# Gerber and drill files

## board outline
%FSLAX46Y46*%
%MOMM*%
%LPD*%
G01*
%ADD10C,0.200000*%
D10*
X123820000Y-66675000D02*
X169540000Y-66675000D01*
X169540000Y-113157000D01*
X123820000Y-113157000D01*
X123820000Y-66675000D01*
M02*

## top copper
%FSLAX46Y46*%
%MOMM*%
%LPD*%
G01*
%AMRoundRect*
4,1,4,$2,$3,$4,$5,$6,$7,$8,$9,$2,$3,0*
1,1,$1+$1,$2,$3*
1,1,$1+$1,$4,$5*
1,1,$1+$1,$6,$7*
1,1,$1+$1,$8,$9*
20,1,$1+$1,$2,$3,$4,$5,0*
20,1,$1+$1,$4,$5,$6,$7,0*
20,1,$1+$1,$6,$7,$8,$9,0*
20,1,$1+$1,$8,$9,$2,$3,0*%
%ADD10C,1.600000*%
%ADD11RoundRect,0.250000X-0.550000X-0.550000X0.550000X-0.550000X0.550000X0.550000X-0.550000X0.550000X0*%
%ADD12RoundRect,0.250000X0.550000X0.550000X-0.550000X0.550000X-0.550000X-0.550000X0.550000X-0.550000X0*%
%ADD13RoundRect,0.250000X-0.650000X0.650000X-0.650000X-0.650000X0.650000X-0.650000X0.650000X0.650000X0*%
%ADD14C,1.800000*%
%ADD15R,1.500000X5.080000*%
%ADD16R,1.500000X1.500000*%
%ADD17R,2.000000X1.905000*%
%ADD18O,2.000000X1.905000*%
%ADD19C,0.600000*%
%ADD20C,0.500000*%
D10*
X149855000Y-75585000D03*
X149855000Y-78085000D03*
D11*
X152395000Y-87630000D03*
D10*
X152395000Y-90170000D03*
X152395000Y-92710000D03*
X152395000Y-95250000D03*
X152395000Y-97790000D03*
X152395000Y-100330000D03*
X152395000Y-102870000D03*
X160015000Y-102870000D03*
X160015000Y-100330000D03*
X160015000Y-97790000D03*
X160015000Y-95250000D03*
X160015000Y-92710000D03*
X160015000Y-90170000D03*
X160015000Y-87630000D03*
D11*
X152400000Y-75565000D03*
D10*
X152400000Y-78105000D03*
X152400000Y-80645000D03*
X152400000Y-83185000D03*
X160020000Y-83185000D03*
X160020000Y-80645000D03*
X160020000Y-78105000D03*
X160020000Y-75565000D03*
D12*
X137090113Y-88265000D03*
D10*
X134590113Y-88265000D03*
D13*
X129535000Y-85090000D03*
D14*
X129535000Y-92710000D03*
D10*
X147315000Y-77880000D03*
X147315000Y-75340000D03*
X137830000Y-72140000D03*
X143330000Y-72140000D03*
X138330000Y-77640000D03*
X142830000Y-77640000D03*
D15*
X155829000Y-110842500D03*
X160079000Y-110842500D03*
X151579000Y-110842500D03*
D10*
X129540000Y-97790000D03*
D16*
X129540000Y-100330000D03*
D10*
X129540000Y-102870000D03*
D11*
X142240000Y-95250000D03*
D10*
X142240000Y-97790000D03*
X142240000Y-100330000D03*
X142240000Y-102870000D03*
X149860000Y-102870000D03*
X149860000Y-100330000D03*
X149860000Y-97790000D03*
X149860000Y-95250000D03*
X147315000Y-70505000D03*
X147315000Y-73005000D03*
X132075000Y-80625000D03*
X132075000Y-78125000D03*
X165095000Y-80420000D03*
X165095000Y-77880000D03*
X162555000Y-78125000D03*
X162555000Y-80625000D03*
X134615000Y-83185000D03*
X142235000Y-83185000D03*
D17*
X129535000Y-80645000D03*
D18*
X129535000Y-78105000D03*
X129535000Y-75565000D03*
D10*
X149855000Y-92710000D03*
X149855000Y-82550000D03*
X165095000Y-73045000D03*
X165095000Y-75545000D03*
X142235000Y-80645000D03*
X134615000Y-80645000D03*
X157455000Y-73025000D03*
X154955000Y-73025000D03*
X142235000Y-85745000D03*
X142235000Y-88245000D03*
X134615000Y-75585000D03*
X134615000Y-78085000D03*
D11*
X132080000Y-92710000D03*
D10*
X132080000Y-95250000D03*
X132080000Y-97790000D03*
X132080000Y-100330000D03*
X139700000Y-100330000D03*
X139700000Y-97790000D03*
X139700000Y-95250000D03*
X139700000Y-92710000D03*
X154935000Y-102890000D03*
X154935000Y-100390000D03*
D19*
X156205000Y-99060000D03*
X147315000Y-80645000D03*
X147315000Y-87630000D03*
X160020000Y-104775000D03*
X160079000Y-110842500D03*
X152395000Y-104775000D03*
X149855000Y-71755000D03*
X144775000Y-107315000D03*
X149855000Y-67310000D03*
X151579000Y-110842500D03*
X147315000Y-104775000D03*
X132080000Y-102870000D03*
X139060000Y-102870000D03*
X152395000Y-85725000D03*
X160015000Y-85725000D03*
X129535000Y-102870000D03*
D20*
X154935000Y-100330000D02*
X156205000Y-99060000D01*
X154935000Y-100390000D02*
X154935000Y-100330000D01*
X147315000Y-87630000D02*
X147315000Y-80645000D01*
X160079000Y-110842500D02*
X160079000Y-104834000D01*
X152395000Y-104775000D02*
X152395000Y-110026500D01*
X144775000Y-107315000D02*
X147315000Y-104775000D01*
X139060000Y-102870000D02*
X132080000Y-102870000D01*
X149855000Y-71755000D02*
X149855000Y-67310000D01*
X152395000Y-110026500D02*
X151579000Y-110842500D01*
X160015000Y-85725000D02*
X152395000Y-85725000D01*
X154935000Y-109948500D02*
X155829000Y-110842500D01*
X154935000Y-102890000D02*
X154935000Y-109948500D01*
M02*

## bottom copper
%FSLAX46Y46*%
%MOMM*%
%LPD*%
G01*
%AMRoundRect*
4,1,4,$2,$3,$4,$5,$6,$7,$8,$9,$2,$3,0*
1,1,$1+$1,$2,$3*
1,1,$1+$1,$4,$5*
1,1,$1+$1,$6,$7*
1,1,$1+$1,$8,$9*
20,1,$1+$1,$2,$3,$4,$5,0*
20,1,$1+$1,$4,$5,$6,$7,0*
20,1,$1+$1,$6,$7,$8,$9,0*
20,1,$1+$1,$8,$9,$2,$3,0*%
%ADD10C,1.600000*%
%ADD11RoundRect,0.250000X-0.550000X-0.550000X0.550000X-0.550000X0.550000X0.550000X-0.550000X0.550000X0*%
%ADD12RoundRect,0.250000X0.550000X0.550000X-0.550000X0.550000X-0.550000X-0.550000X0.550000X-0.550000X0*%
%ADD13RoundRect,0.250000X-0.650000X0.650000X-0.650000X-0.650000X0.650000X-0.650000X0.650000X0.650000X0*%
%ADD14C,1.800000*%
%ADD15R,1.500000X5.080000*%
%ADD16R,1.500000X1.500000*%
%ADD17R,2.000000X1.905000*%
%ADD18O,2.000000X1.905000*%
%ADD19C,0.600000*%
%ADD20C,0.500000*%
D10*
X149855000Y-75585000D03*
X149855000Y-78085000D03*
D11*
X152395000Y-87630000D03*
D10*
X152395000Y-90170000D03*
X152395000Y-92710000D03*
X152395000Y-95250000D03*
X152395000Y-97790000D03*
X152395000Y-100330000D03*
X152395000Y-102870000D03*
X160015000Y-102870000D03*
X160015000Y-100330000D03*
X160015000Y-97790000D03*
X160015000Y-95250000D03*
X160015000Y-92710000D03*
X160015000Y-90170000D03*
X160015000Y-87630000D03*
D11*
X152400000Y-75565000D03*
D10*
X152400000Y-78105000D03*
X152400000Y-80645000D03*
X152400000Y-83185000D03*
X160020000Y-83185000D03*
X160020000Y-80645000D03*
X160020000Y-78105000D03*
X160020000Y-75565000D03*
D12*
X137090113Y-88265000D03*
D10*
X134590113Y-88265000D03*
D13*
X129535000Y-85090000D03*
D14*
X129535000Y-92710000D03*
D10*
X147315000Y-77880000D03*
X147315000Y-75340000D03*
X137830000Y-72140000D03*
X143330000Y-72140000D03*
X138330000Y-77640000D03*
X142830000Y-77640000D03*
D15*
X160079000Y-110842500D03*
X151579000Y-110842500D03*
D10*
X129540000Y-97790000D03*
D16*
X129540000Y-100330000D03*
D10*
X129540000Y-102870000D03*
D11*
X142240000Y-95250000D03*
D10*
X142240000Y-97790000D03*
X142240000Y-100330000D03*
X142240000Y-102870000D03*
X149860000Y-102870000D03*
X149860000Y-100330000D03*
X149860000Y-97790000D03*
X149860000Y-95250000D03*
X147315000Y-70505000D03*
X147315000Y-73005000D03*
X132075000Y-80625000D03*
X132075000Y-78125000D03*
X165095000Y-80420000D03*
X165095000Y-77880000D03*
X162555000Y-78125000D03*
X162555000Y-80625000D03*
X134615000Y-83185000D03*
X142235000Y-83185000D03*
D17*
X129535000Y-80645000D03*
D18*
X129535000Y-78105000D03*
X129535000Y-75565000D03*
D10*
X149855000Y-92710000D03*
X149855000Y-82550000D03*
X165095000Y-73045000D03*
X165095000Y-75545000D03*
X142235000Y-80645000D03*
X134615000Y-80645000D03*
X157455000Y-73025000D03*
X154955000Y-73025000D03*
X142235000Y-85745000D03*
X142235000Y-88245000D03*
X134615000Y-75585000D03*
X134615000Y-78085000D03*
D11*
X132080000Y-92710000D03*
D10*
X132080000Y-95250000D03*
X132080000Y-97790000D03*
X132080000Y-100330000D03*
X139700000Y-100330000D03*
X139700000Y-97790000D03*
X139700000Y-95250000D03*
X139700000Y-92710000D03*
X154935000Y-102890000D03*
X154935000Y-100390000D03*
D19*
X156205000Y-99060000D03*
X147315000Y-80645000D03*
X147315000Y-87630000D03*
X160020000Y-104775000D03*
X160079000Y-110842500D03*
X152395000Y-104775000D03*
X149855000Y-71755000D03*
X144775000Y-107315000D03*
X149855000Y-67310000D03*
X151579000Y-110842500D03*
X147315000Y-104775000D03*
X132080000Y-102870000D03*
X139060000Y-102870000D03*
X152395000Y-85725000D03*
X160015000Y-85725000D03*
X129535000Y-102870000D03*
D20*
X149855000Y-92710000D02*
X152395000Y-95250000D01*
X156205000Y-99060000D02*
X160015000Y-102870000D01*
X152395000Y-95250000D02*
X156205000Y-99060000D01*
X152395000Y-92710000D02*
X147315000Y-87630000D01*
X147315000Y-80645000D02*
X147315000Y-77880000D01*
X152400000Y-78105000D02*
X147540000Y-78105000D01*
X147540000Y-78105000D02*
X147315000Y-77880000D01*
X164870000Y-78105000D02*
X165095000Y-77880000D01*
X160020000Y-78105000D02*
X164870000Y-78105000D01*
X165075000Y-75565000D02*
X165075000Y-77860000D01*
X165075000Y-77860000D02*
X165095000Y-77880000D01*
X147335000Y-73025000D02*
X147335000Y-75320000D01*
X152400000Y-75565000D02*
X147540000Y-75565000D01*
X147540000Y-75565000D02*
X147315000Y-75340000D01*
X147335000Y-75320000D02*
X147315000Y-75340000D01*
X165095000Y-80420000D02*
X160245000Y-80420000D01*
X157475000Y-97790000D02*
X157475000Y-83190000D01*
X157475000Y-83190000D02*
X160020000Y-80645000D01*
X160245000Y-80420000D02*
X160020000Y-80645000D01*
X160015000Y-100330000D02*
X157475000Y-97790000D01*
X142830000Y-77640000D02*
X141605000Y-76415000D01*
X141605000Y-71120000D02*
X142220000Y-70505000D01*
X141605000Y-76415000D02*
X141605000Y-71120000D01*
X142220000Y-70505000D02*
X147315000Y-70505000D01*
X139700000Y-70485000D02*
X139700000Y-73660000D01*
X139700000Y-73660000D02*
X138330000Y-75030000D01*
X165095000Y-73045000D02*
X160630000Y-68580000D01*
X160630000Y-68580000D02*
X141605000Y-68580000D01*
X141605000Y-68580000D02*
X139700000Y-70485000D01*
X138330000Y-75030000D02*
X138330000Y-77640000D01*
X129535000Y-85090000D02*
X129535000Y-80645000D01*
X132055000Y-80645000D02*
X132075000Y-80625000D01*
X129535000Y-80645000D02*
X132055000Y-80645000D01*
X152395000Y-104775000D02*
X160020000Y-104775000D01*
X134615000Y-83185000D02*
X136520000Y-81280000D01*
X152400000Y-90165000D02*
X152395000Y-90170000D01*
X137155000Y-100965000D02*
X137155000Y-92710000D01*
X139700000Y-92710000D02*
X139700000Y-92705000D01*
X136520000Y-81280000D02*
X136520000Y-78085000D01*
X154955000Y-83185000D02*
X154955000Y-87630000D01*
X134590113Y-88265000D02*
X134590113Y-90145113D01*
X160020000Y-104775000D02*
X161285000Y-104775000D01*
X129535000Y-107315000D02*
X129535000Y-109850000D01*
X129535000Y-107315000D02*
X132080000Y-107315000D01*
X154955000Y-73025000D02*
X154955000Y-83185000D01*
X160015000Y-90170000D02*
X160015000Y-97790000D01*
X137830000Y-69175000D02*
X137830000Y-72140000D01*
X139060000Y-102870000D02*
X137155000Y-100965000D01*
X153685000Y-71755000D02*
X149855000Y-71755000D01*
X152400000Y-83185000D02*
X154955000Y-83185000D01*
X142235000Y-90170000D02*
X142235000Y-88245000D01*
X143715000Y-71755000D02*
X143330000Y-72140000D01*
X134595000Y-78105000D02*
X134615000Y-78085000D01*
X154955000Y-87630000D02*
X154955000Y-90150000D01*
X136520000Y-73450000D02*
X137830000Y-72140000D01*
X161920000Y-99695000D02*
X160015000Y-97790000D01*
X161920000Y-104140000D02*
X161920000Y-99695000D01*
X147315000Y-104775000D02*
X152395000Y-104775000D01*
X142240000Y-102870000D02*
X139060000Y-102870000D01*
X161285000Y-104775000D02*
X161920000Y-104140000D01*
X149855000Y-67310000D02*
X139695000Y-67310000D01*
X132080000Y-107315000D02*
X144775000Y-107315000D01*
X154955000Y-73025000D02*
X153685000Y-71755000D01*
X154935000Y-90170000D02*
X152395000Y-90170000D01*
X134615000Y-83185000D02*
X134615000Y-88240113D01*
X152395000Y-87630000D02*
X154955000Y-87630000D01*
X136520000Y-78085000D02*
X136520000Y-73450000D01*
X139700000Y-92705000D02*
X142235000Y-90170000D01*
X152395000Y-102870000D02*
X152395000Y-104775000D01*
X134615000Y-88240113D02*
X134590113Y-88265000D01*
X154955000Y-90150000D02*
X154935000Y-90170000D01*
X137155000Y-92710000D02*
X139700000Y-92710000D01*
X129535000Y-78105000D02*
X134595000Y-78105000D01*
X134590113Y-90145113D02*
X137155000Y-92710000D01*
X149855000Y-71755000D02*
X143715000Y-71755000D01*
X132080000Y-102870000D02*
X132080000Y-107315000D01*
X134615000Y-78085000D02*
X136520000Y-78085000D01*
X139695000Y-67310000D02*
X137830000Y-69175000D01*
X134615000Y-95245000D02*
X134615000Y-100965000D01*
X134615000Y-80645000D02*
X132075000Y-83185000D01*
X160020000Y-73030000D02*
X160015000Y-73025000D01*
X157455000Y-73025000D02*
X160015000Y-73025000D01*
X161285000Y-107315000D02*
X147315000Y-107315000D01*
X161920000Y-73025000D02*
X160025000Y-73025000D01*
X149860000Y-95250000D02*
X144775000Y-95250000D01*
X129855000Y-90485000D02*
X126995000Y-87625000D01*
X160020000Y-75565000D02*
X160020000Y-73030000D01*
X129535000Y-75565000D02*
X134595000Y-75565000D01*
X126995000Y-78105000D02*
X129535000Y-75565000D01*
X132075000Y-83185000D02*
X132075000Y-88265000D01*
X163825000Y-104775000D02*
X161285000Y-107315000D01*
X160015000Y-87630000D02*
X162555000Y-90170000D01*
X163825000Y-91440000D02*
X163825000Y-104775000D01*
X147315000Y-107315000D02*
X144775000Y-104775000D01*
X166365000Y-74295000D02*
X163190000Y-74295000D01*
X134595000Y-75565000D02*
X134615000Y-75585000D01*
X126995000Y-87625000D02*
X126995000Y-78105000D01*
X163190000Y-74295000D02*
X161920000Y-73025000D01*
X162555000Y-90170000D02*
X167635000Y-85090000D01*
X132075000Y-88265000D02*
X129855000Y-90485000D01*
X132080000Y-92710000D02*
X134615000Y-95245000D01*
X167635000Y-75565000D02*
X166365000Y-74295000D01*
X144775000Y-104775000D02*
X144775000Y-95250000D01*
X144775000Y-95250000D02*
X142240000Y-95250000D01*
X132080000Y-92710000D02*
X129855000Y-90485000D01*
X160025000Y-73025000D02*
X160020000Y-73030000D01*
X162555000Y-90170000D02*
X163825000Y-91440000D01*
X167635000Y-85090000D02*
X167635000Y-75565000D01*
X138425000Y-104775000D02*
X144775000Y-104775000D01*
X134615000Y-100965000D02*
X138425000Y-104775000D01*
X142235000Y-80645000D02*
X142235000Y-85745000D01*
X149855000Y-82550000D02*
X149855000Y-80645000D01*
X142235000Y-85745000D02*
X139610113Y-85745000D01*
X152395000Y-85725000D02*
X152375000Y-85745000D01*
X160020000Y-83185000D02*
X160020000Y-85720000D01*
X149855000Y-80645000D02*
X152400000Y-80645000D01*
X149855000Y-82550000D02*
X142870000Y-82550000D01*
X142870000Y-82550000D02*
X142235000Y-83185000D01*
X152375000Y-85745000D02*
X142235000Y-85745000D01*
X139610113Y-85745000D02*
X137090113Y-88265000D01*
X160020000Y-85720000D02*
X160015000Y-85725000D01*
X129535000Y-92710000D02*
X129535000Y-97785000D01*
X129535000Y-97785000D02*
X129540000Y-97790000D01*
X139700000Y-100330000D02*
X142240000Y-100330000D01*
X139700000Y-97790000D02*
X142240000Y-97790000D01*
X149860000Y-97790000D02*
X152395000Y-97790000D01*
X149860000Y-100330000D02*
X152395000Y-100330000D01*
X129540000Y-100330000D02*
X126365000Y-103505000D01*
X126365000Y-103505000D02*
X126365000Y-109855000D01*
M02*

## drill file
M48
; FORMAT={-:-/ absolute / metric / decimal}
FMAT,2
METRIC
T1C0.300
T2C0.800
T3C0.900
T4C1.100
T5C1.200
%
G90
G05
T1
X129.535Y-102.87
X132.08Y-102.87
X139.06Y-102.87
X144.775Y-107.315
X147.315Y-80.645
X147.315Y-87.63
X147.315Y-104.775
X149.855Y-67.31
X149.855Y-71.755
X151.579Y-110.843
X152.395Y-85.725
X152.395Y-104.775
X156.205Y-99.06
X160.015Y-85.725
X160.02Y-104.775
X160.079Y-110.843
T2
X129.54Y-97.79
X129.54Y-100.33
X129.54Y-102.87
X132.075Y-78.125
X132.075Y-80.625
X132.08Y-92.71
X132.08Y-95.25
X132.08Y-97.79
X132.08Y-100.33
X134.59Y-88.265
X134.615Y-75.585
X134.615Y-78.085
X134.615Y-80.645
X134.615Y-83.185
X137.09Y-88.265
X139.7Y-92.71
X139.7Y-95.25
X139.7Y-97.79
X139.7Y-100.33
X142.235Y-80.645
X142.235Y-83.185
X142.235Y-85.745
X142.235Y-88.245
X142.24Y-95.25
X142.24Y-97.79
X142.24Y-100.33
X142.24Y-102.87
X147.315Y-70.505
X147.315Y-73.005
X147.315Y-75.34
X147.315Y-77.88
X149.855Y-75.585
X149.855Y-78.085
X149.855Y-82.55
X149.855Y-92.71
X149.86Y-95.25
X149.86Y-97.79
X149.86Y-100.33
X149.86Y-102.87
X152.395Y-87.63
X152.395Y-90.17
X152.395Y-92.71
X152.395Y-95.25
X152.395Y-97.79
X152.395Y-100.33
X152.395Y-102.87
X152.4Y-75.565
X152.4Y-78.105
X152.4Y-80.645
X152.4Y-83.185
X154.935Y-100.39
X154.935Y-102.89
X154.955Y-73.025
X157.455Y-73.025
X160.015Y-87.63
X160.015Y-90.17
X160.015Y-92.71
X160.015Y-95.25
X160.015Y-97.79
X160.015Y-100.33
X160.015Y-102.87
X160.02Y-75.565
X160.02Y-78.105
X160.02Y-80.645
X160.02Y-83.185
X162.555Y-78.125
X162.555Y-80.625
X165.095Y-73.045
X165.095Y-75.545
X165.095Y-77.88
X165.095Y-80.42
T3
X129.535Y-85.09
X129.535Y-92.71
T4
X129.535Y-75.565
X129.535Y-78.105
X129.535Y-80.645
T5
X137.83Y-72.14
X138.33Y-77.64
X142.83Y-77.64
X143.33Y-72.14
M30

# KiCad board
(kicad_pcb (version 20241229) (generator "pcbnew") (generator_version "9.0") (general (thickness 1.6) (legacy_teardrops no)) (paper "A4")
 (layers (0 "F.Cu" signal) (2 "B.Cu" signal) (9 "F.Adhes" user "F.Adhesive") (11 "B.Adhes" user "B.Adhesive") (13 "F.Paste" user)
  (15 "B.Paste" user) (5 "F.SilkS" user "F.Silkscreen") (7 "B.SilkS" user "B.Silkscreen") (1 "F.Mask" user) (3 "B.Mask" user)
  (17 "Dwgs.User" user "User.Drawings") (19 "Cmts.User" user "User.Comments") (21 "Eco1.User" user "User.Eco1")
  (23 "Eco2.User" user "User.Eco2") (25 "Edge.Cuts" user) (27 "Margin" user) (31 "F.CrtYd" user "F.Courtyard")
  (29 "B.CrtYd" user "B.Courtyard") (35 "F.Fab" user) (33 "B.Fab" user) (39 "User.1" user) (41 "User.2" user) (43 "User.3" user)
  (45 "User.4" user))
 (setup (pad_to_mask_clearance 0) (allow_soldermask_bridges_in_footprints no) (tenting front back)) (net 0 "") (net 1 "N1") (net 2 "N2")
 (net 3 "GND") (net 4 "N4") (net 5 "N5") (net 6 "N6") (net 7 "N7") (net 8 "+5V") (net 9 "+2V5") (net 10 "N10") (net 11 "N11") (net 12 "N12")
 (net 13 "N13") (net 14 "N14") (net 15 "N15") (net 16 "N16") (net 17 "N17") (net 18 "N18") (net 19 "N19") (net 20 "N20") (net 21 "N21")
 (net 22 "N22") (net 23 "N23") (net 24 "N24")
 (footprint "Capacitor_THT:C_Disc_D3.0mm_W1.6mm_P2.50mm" (layer "F.Cu") (at 149.855 75.585 -90)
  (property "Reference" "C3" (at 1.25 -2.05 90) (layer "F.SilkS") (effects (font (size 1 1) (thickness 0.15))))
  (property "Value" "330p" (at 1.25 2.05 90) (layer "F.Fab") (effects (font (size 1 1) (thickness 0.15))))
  (pad "1" thru_hole circle (at 0 0 270) (size 1.6 1.6) (drill 0.8) (layers "*.Cu" "*.Mask") (remove_unused_layers no) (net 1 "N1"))
  (pad "2" thru_hole circle (at 2.5 0 270) (size 1.6 1.6) (drill 0.8) (layers "*.Cu" "*.Mask") (remove_unused_layers no) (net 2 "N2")))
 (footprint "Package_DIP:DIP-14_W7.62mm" (layer "F.Cu") (at 152.395 87.63)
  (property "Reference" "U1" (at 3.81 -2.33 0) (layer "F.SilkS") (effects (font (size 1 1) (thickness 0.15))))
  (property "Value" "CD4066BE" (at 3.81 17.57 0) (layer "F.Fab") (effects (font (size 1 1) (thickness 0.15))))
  (pad "1" thru_hole roundrect (at 0 0) (size 1.6 1.6) (drill 0.8) (layers "*.Cu" "*.Mask") (remove_unused_layers no)
   (roundrect_rratio 0.15625) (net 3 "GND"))
  (pad "2" thru_hole circle (at 0 2.54) (size 1.6 1.6) (drill 0.8) (layers "*.Cu" "*.Mask") (remove_unused_layers no) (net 3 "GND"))
  (pad "3" thru_hole circle (at 0 5.08) (size 1.6 1.6) (drill 0.8) (layers "*.Cu" "*.Mask") (remove_unused_layers no) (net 2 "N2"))
  (pad "4" thru_hole circle (at 0 7.62) (size 1.6 1.6) (drill 0.8) (layers "*.Cu" "*.Mask") (remove_unused_layers no) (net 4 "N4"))
  (pad "5" thru_hole circle (at 0 10.16) (size 1.6 1.6) (drill 0.8) (layers "*.Cu" "*.Mask") (remove_unused_layers no) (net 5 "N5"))
  (pad "6" thru_hole circle (at 0 12.7) (size 1.6 1.6) (drill 0.8) (layers "*.Cu" "*.Mask") (remove_unused_layers no) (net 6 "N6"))
  (pad "7" thru_hole circle (at 0 15.24) (size 1.6 1.6) (drill 0.8) (layers "*.Cu" "*.Mask") (remove_unused_layers no) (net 3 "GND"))
  (pad "8" thru_hole circle (at 7.62 15.24) (size 1.6 1.6) (drill 0.8) (layers "*.Cu" "*.Mask") (remove_unused_layers no) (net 4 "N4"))
  (pad "9" thru_hole circle (at 7.62 12.7) (size 1.6 1.6) (drill 0.8) (layers "*.Cu" "*.Mask") (remove_unused_layers no) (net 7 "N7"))
  (pad "10" thru_hole circle (at 7.62 10.16) (size 1.6 1.6) (drill 0.8) (layers "*.Cu" "*.Mask") (remove_unused_layers no) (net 3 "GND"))
  (pad "11" thru_hole circle (at 7.62 7.62) (size 1.6 1.6) (drill 0.8) (layers "*.Cu" "*.Mask") (remove_unused_layers no) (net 3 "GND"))
  (pad "12" thru_hole circle (at 7.62 5.08) (size 1.6 1.6) (drill 0.8) (layers "*.Cu" "*.Mask") (remove_unused_layers no) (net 3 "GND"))
  (pad "13" thru_hole circle (at 7.62 2.54) (size 1.6 1.6) (drill 0.8) (layers "*.Cu" "*.Mask") (remove_unused_layers no) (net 3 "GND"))
  (pad "14" thru_hole circle (at 7.62 0) (size 1.6 1.6) (drill 0.8) (layers "*.Cu" "*.Mask") (remove_unused_layers no) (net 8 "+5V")))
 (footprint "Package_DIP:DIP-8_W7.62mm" (layer "F.Cu") (at 152.4 75.565)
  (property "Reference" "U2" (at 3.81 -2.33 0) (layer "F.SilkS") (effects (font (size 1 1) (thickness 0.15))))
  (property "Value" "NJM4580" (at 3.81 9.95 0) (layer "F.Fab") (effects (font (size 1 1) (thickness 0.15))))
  (pad "1" thru_hole roundrect (at 0 0) (size 1.6 1.6) (drill 0.8) (layers "*.Cu" "*.Mask") (remove_unused_layers no)
   (roundrect_rratio 0.15625) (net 1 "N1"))
  (pad "2" thru_hole circle (at 0 2.54) (size 1.6 1.6) (drill 0.8) (layers "*.Cu" "*.Mask") (remove_unused_layers no) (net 2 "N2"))
  (pad "3" thru_hole circle (at 0 5.08) (size 1.6 1.6) (drill 0.8) (layers "*.Cu" "*.Mask") (remove_unused_layers no) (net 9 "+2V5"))
  (pad "4" thru_hole circle (at 0 7.62) (size 1.6 1.6) (drill 0.8) (layers "*.Cu" "*.Mask") (remove_unused_layers no) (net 3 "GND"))
  (pad "5" thru_hole circle (at 7.62 7.62) (size 1.6 1.6) (drill 0.8) (layers "*.Cu" "*.Mask") (remove_unused_layers no) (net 9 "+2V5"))
  (pad "6" thru_hole circle (at 7.62 5.08) (size 1.6 1.6) (drill 0.8) (layers "*.Cu" "*.Mask") (remove_unused_layers no) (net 7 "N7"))
  (pad "7" thru_hole circle (at 7.62 2.54) (size 1.6 1.6) (drill 0.8) (layers "*.Cu" "*.Mask") (remove_unused_layers no) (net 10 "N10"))
  (pad "8" thru_hole circle (at 7.62 0) (size 1.6 1.6) (drill 0.8) (layers "*.Cu" "*.Mask") (remove_unused_layers no) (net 8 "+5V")))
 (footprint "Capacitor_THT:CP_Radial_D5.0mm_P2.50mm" (layer "F.Cu") (at 137.090113 88.265 180)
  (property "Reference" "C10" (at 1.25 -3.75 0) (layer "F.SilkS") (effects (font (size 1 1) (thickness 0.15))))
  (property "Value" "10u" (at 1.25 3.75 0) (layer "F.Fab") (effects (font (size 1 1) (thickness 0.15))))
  (pad "1" thru_hole roundrect (at 0 0 180) (size 1.6 1.6) (drill 0.8) (layers "*.Cu" "*.Mask") (remove_unused_layers no)
   (roundrect_rratio 0.15625) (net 9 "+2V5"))
  (pad "2" thru_hole circle (at 2.5 0 180) (size 1.6 1.6) (drill 0.8) (layers "*.Cu" "*.Mask") (remove_unused_layers no) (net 3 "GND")))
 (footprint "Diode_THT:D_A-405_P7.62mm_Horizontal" (layer "F.Cu") (at 129.535 85.09 -90)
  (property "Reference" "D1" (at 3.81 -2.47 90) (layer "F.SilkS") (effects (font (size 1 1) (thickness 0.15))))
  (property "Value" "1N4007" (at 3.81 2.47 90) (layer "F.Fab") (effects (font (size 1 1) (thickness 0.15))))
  (pad "1" thru_hole roundrect (at 0 0 270) (size 1.8 1.8) (drill 0.9) (layers "*.Cu" "*.Mask") (remove_unused_layers no)
   (roundrect_rratio 0.138889) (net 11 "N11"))
  (pad "2" thru_hole circle (at 7.62 0 270) (size 1.8 1.8) (drill 0.9) (layers "*.Cu" "*.Mask") (remove_unused_layers no) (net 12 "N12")))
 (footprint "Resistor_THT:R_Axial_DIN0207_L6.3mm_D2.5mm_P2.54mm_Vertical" (layer "F.Cu") (at 147.315 77.88 90)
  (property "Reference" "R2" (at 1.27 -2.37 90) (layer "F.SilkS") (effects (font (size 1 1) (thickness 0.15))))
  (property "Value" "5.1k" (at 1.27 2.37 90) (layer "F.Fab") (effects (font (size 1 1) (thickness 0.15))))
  (pad "1" thru_hole circle (at 0 0 90) (size 1.6 1.6) (drill 0.8) (layers "*.Cu" "*.Mask") (remove_unused_layers no) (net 2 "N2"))
  (pad "2" thru_hole circle (at 2.54 0 90) (size 1.6 1.6) (drill 0.8) (layers "*.Cu" "*.Mask") (remove_unused_layers no) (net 1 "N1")))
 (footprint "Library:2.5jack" (layer "F.Cu") (at 140.33 72.39)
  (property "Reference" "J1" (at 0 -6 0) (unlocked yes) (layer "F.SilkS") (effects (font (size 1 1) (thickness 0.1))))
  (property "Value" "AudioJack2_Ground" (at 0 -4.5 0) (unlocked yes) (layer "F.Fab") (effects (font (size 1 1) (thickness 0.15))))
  (pad "G" thru_hole circle (at -2.5 -0.25) (size 1.6 1.6) (drill 1.2) (layers "*.Cu" "*.Mask") (remove_unused_layers no) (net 3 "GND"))
  (pad "G" thru_hole circle (at 3 -0.25) (size 1.6 1.6) (drill 1.2) (layers "*.Cu" "*.Mask") (remove_unused_layers no) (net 3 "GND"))
  (pad "S" thru_hole circle (at -2 5.25) (size 1.6 1.6) (drill 1.2) (layers "*.Cu" "*.Mask") (remove_unused_layers no) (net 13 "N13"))
  (pad "T" thru_hole circle (at 2.5 5.25) (size 1.6 1.6) (drill 1.2) (layers "*.Cu" "*.Mask") (remove_unused_layers no) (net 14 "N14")))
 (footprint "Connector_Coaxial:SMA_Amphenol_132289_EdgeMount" (layer "F.Cu") (at 155.829 110.8425 -90)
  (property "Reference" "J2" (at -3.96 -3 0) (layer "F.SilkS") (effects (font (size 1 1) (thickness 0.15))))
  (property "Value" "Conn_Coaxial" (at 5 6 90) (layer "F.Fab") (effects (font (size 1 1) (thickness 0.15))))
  (pad "1" smd rect (at 0 0) (size 1.5 5.08) (layers "F.Cu" "F.Mask" "F.Paste") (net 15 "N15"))
  (pad "2" smd rect (at 0 -4.25) (size 1.5 5.08) (layers "F.Cu" "F.Mask" "F.Paste") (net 3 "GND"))
  (pad "2" smd rect (at 0 -4.25) (size 1.5 5.08) (layers "B.Cu" "B.Mask" "B.Paste") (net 3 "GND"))
  (pad "2" smd rect (at 0 4.25) (size 1.5 5.08) (layers "F.Cu" "F.Mask" "F.Paste") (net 3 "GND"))
  (pad "2" smd rect (at 0 4.25) (size 1.5 5.08) (layers "B.Cu" "B.Mask" "B.Paste") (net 3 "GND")))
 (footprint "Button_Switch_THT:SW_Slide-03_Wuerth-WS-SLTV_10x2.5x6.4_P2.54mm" (layer "F.Cu") (at 129.54 100.33 -90)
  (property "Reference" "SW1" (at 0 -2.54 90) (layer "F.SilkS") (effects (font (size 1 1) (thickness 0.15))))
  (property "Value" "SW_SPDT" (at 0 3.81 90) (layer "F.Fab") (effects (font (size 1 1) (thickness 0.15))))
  (pad "1" thru_hole circle (at -2.54 0 270) (size 1.6 1.6) (drill 0.8) (layers "*.Cu" "*.Mask") (remove_unused_layers no) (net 12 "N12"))
  (pad "2" thru_hole rect (at 0 0 270) (size 1.5 1.5) (drill 0.8) (layers "*.Cu" "*.Mask") (remove_unused_layers no) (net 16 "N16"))
  (pad "3" thru_hole circle (at 2.54 0 270) (size 1.6 1.6) (drill 0.8) (layers "*.Cu" "*.Mask") (remove_unused_layers no) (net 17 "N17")))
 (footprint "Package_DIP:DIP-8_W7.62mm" (layer "F.Cu") (at 142.24 95.25)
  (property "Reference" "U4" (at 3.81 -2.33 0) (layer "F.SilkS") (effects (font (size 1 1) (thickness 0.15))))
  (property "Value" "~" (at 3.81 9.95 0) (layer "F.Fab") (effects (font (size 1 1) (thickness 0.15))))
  (pad "1" thru_hole roundrect (at 0 0) (size 1.6 1.6) (drill 0.8) (layers "*.Cu" "*.Mask") (remove_unused_layers no)
   (roundrect_rratio 0.15625) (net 8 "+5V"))
  (pad "2" thru_hole circle (at 0 2.54) (size 1.6 1.6) (drill 0.8) (layers "*.Cu" "*.Mask") (remove_unused_layers no) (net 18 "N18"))
  (pad "3" thru_hole circle (at 0 5.08) (size 1.6 1.6) (drill 0.8) (layers "*.Cu" "*.Mask") (remove_unused_layers no) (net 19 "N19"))
  (pad "4" thru_hole circle (at 0 7.62) (size 1.6 1.6) (drill 0.8) (layers "*.Cu" "*.Mask") (remove_unused_layers no) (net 3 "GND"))
  (pad "5" thru_hole circle (at 7.62 7.62) (size 1.6 1.6) (drill 0.8) (layers "*.Cu" "*.Mask") (remove_unused_layers no) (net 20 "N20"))
  (pad "6" thru_hole circle (at 7.62 5.08) (size 1.6 1.6) (drill 0.8) (layers "*.Cu" "*.Mask") (remove_unused_layers no) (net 6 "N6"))
  (pad "7" thru_hole circle (at 7.62 2.54) (size 1.6 1.6) (drill 0.8) (layers "*.Cu" "*.Mask") (remove_unused_layers no) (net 5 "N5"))
  (pad "8" thru_hole circle (at 7.62 0) (size 1.6 1.6) (drill 0.8) (layers "*.Cu" "*.Mask") (remove_unused_layers no) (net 8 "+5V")))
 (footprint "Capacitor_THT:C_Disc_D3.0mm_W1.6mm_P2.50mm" (layer "F.Cu") (at 147.315 70.505 -90)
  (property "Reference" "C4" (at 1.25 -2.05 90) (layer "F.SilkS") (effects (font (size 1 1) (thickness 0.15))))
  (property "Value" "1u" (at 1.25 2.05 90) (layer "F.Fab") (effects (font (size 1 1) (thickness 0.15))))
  (pad "1" thru_hole circle (at 0 0 270) (size 1.6 1.6) (drill 0.8) (layers "*.Cu" "*.Mask") (remove_unused_layers no) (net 14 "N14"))
  (pad "2" thru_hole circle (at 2.5 0 270) (size 1.6 1.6) (drill 0.8) (layers "*.Cu" "*.Mask") (remove_unused_layers no) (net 1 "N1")))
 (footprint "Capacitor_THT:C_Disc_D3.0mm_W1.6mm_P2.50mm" (layer "F.Cu") (at 132.075 80.625 90)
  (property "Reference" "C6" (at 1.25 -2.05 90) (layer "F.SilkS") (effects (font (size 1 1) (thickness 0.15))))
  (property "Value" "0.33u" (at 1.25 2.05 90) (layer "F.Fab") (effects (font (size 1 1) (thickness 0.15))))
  (pad "1" thru_hole circle (at 0 0 90) (size 1.6 1.6) (drill 0.8) (layers "*.Cu" "*.Mask") (remove_unused_layers no) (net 11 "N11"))
  (pad "2" thru_hole circle (at 2.5 0 90) (size 1.6 1.6) (drill 0.8) (layers "*.Cu" "*.Mask") (remove_unused_layers no) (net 3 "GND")))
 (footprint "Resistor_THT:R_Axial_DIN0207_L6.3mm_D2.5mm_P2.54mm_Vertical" (layer "F.Cu") (at 165.095 80.42 90)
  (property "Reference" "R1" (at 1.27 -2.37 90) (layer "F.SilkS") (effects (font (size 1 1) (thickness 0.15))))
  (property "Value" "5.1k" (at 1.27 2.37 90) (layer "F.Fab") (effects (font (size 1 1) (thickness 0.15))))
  (pad "1" thru_hole circle (at 0 0 90) (size 1.6 1.6) (drill 0.8) (layers "*.Cu" "*.Mask") (remove_unused_layers no) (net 7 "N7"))
  (pad "2" thru_hole circle (at 2.54 0 90) (size 1.6 1.6) (drill 0.8) (layers "*.Cu" "*.Mask") (remove_unused_layers no) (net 10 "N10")))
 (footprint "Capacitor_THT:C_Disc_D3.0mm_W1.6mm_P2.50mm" (layer "F.Cu") (at 162.555 78.125 -90)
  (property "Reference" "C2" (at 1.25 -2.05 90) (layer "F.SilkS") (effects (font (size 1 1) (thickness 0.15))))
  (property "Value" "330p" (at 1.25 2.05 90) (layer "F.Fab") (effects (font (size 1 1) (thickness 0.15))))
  (pad "1" thru_hole circle (at 0 0 270) (size 1.6 1.6) (drill 0.8) (layers "*.Cu" "*.Mask") (remove_unused_layers no) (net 10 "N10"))
  (pad "2" thru_hole circle (at 2.5 0 270) (size 1.6 1.6) (drill 0.8) (layers "*.Cu" "*.Mask") (remove_unused_layers no) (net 7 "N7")))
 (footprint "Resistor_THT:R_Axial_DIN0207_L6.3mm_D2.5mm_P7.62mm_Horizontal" (layer "F.Cu") (at 134.615 83.185)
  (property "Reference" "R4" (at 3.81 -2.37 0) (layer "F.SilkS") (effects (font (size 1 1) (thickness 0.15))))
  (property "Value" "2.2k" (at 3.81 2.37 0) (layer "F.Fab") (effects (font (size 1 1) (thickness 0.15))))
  (pad "1" thru_hole circle (at 0 0) (size 1.6 1.6) (drill 0.8) (layers "*.Cu" "*.Mask") (remove_unused_layers no) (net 3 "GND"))
  (pad "2" thru_hole circle (at 7.62 0) (size 1.6 1.6) (drill 0.8) (layers "*.Cu" "*.Mask") (remove_unused_layers no) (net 9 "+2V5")))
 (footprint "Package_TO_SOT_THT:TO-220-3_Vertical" (layer "F.Cu") (at 129.535 80.645 90)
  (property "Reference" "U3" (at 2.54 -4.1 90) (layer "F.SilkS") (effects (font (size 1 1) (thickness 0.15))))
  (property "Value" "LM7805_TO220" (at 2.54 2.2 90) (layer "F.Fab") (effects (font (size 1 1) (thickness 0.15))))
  (pad "1" thru_hole rect (at 0 0 90) (size 1.905 2) (drill 1.1) (layers "*.Cu" "*.Mask") (remove_unused_layers no) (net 11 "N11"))
  (pad "2" thru_hole oval (at 2.54 0 90) (size 1.905 2) (drill 1.1) (layers "*.Cu" "*.Mask") (remove_unused_layers no) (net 3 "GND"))
  (pad "3" thru_hole oval (at 5.08 0 90) (size 1.905 2) (drill 1.1) (layers "*.Cu" "*.Mask") (remove_unused_layers no) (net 8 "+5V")))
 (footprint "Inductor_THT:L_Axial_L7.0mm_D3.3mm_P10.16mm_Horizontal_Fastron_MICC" (layer "F.Cu") (at 149.855 92.71 90)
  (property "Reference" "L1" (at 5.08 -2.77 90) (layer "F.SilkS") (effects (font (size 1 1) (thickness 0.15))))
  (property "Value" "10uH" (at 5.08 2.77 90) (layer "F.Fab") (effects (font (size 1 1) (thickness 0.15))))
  (pad "1" thru_hole circle (at 0 0 90) (size 1.6 1.6) (drill 0.8) (layers "*.Cu" "*.Mask") (remove_unused_layers no) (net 4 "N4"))
  (pad "2" thru_hole circle (at 10.16 0 90) (size 1.6 1.6) (drill 0.8) (layers "*.Cu" "*.Mask") (remove_unused_layers no) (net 9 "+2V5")))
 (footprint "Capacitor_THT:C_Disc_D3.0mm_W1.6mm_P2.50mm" (layer "F.Cu") (at 165.095 73.045 -90)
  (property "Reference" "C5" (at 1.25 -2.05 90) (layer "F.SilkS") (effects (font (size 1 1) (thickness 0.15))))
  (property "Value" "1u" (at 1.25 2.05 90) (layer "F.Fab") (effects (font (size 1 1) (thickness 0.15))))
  (pad "1" thru_hole circle (at 0 0 270) (size 1.6 1.6) (drill 0.8) (layers "*.Cu" "*.Mask") (remove_unused_layers no) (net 13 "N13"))
  (pad "2" thru_hole circle (at 2.5 0 270) (size 1.6 1.6) (drill 0.8) (layers "*.Cu" "*.Mask") (remove_unused_layers no) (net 10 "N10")))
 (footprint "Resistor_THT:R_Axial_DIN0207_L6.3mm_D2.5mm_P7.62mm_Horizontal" (layer "F.Cu") (at 142.235 80.645 180)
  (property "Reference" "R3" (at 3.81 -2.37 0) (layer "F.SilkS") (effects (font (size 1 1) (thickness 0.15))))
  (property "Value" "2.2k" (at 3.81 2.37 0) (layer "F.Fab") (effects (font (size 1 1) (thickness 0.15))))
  (pad "1" thru_hole circle (at 0 0 180) (size 1.6 1.6) (drill 0.8) (layers "*.Cu" "*.Mask") (remove_unused_layers no) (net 9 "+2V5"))
  (pad "2" thru_hole circle (at 7.62 0 180) (size 1.6 1.6) (drill 0.8) (layers "*.Cu" "*.Mask") (remove_unused_layers no) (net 8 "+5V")))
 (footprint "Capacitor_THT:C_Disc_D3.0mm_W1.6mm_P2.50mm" (layer "F.Cu") (at 157.455 73.025 180)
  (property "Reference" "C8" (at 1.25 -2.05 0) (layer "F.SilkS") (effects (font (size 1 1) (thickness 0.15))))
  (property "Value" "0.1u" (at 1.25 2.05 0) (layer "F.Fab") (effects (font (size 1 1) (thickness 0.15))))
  (pad "1" thru_hole circle (at 0 0 180) (size 1.6 1.6) (drill 0.8) (layers "*.Cu" "*.Mask") (remove_unused_layers no) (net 8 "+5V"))
  (pad "2" thru_hole circle (at 2.5 0 180) (size 1.6 1.6) (drill 0.8) (layers "*.Cu" "*.Mask") (remove_unused_layers no) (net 3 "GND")))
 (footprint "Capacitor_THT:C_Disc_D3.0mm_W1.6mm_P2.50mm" (layer "F.Cu") (at 142.235 85.745 -90)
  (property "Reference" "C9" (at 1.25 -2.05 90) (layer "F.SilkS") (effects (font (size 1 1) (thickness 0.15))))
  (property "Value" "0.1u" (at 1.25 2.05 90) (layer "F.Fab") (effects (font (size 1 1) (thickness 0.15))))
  (pad "1" thru_hole circle (at 0 0 270) (size 1.6 1.6) (drill 0.8) (layers "*.Cu" "*.Mask") (remove_unused_layers no) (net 9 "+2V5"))
  (pad "2" thru_hole circle (at 2.5 0 270) (size 1.6 1.6) (drill 0.8) (layers "*.Cu" "*.Mask") (remove_unused_layers no) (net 3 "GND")))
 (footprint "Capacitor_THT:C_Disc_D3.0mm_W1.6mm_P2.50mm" (layer "F.Cu") (at 134.615 75.585 -90)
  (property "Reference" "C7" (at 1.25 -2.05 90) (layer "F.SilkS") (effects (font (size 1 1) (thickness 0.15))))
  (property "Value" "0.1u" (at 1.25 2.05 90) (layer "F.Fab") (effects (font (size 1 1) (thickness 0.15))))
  (pad "1" thru_hole circle (at 0 0 270) (size 1.6 1.6) (drill 0.8) (layers "*.Cu" "*.Mask") (remove_unused_layers no) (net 8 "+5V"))
  (pad "2" thru_hole circle (at 2.5 0 270) (size 1.6 1.6) (drill 0.8) (layers "*.Cu" "*.Mask") (remove_unused_layers no) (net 3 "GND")))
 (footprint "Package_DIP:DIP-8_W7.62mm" (layer "F.Cu") (at 132.08 92.71)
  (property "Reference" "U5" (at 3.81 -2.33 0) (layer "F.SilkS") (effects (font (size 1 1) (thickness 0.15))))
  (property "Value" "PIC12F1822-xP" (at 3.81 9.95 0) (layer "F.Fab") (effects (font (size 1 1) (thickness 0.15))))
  (pad "1" thru_hole roundrect (at 0 0) (size 1.6 1.6) (drill 0.8) (layers "*.Cu" "*.Mask") (remove_unused_layers no)
   (roundrect_rratio 0.15625) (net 8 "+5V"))
  (pad "2" thru_hole circle (at 0 2.54) (size 1.6 1.6) (drill 0.8) (layers "*.Cu" "*.Mask") (remove_unused_layers no) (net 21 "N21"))
  (pad "3" thru_hole circle (at 0 5.08) (size 1.6 1.6) (drill 0.8) (layers "*.Cu" "*.Mask") (remove_unused_layers no) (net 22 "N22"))
  (pad "4" thru_hole circle (at 0 7.62) (size 1.6 1.6) (drill 0.8) (layers "*.Cu" "*.Mask") (remove_unused_layers no) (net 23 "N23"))
  (pad "5" thru_hole circle (at 7.62 7.62) (size 1.6 1.6) (drill 0.8) (layers "*.Cu" "*.Mask") (remove_unused_layers no) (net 19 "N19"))
  (pad "6" thru_hole circle (at 7.62 5.08) (size 1.6 1.6) (drill 0.8) (layers "*.Cu" "*.Mask") (remove_unused_layers no) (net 18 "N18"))
  (pad "7" thru_hole circle (at 7.62 2.54) (size 1.6 1.6) (drill 0.8) (layers "*.Cu" "*.Mask") (remove_unused_layers no) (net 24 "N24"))
  (pad "8" thru_hole circle (at 7.62 0) (size 1.6 1.6) (drill 0.8) (layers "*.Cu" "*.Mask") (remove_unused_layers no) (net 3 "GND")))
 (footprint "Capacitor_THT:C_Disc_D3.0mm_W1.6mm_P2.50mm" (layer "B.Cu") (at 154.935 102.89 90)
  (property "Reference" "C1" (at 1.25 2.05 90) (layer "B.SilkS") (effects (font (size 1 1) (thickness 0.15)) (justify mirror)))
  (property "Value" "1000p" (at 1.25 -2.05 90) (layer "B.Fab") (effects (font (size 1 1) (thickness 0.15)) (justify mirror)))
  (pad "1" thru_hole circle (at 0 0 90) (size 1.6 1.6) (drill 0.8) (layers "*.Cu" "*.Mask") (remove_unused_layers no) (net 15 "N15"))
  (pad "2" thru_hole circle (at 2.5 0 90) (size 1.6 1.6) (drill 0.8) (layers "*.Cu" "*.Mask") (remove_unused_layers no) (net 4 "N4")))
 (gr_rect (start 123.82 66.675) (end 169.54 113.157) (stroke (width 0.2) (type solid)) (fill no) (layer "Edge.Cuts"))
 (segment (start 154.935 100.33) (end 156.205 99.06) (width 0.5) (layer "F.Cu") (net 4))
 (segment (start 154.935 100.39) (end 154.935 100.33) (width 0.5) (layer "F.Cu") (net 4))
 (via (at 156.205 99.06) (size 0.6) (drill 0.3) (layers "F.Cu" "B.Cu") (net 4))
 (segment (start 149.855 92.71) (end 152.395 95.25) (width 0.5) (layer "B.Cu") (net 4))
 (segment (start 156.205 99.06) (end 160.015 102.87) (width 0.5) (layer "B.Cu") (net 4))
 (segment (start 152.395 95.25) (end 156.205 99.06) (width 0.5) (layer "B.Cu") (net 4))
 (segment (start 147.315 87.63) (end 147.315 80.645) (width 0.5) (layer "F.Cu") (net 2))
 (via (at 147.315 80.645) (size 0.6) (drill 0.3) (layers "F.Cu" "B.Cu") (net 2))
 (via (at 147.315 87.63) (size 0.6) (drill 0.3) (layers "F.Cu" "B.Cu") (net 2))
 (segment (start 152.395 92.71) (end 147.315 87.63) (width 0.5) (layer "B.Cu") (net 2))
 (segment (start 147.315 80.645) (end 147.315 77.88) (width 0.5) (layer "B.Cu") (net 2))
 (segment (start 152.4 78.105) (end 147.54 78.105) (width 0.5) (layer "B.Cu") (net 2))
 (segment (start 147.54 78.105) (end 147.315 77.88) (width 0.5) (layer "B.Cu") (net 2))
 (segment (start 164.87 78.105) (end 165.095 77.88) (width 0.5) (layer "B.Cu") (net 10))
 (segment (start 160.02 78.105) (end 164.87 78.105) (width 0.5) (layer "B.Cu") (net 10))
 (segment (start 165.075 75.565) (end 165.075 77.86) (width 0.5) (layer "B.Cu") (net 10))
 (segment (start 165.075 77.86) (end 165.095 77.88) (width 0.5) (layer "B.Cu") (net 10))
 (segment (start 147.335 73.025) (end 147.335 75.32) (width 0.5) (layer "B.Cu") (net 1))
 (segment (start 152.4 75.565) (end 147.54 75.565) (width 0.5) (layer "B.Cu") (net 1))
 (segment (start 147.54 75.565) (end 147.315 75.34) (width 0.5) (layer "B.Cu") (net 1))
 (segment (start 147.335 75.32) (end 147.315 75.34) (width 0.5) (layer "B.Cu") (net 1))
 (segment (start 165.095 80.42) (end 160.245 80.42) (width 0.5) (layer "B.Cu") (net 7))
 (segment (start 157.475 97.79) (end 157.475 83.19) (width 0.5) (layer "B.Cu") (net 7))
 (segment (start 157.475 83.19) (end 160.02 80.645) (width 0.5) (layer "B.Cu") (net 7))
 (segment (start 160.245 80.42) (end 160.02 80.645) (width 0.5) (layer "B.Cu") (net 7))
 (segment (start 160.015 100.33) (end 157.475 97.79) (width 0.5) (layer "B.Cu") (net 7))
 (segment (start 142.83 77.64) (end 141.605 76.415) (width 0.5) (layer "B.Cu") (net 14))
 (segment (start 141.605 71.12) (end 142.22 70.505) (width 0.5) (layer "B.Cu") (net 14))
 (segment (start 141.605 76.415) (end 141.605 71.12) (width 0.5) (layer "B.Cu") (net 14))
 (segment (start 142.22 70.505) (end 147.315 70.505) (width 0.5) (layer "B.Cu") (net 14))
 (segment (start 139.7 70.485) (end 139.7 73.66) (width 0.5) (layer "B.Cu") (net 13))
 (segment (start 139.7 73.66) (end 138.33 75.03) (width 0.5) (layer "B.Cu") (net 13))
 (segment (start 165.095 73.045) (end 160.63 68.58) (width 0.5) (layer "B.Cu") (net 13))
 (segment (start 160.63 68.58) (end 141.605 68.58) (width 0.5) (layer "B.Cu") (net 13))
 (segment (start 141.605 68.58) (end 139.7 70.485) (width 0.5) (layer "B.Cu") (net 13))
 (segment (start 138.33 75.03) (end 138.33 77.64) (width 0.5) (layer "B.Cu") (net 13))
 (segment (start 129.535 85.09) (end 129.535 80.645) (width 0.5) (layer "B.Cu") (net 11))
 (segment (start 132.055 80.645) (end 132.075 80.625) (width 0.5) (layer "B.Cu") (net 11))
 (segment (start 129.535 80.645) (end 132.055 80.645) (width 0.5) (layer "B.Cu") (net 11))
 (segment (start 160.079 110.8425) (end 160.079 104.834) (width 0.5) (layer "F.Cu") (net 3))
 (segment (start 152.395 104.775) (end 152.395 110.0265) (width 0.5) (layer "F.Cu") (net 3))
 (segment (start 144.775 107.315) (end 147.315 104.775) (width 0.5) (layer "F.Cu") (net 3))
 (segment (start 139.06 102.87) (end 132.08 102.87) (width 0.5) (layer "F.Cu") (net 3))
 (segment (start 149.855 71.755) (end 149.855 67.31) (width 0.5) (layer "F.Cu") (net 3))
 (segment (start 152.395 110.0265) (end 151.579 110.8425) (width 0.5) (layer "F.Cu") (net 3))
 (via (at 160.02 104.775) (size 0.6) (drill 0.3) (layers "F.Cu" "B.Cu") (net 3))
 (via (at 160.079 110.8425) (size 0.6) (drill 0.3) (layers "F.Cu" "B.Cu") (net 3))
 (via (at 152.395 104.775) (size 0.6) (drill 0.3) (layers "F.Cu" "B.Cu") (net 3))
 (via (at 149.855 71.755) (size 0.6) (drill 0.3) (layers "F.Cu" "B.Cu") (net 3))
 (via (at 144.775 107.315) (size 0.6) (drill 0.3) (layers "F.Cu" "B.Cu") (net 3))
 (via (at 149.855 67.31) (size 0.6) (drill 0.3) (layers "F.Cu" "B.Cu") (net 3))
 (via (at 151.579 110.8425) (size 0.6) (drill 0.3) (layers "F.Cu" "B.Cu") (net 3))
 (via (at 147.315 104.775) (size 0.6) (drill 0.3) (layers "F.Cu" "B.Cu") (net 3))
 (via (at 132.08 102.87) (size 0.6) (drill 0.3) (layers "F.Cu" "B.Cu") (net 3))
 (via (at 139.06 102.87) (size 0.6) (drill 0.3) (layers "F.Cu" "B.Cu") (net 3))
 (segment (start 152.395 104.775) (end 160.02 104.775) (width 0.5) (layer "B.Cu") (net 3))
 (segment (start 134.615 83.185) (end 136.52 81.28) (width 0.5) (layer "B.Cu") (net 3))
 (segment (start 152.4 90.165) (end 152.395 90.17) (width 0.5) (layer "B.Cu") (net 3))
 (segment (start 137.155 100.965) (end 137.155 92.71) (width 0.5) (layer "B.Cu") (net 3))
 (segment (start 139.7 92.71) (end 139.7 92.705) (width 0.5) (layer "B.Cu") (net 3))
 (segment (start 136.52 81.28) (end 136.52 78.085) (width 0.5) (layer "B.Cu") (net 3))
 (segment (start 154.955 83.185) (end 154.955 87.63) (width 0.5) (layer "B.Cu") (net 3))
 (segment (start 134.590113 88.265) (end 134.590113 90.145113) (width 0.5) (layer "B.Cu") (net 3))
 (segment (start 160.02 104.775) (end 161.285 104.775) (width 0.5) (layer "B.Cu") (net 3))
 (segment (start 129.535 107.315) (end 129.535 109.85) (width 0.5) (layer "B.Cu") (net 3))
 (segment (start 129.535 107.315) (end 132.08 107.315) (width 0.5) (layer "B.Cu") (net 3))
 (segment (start 154.955 73.025) (end 154.955 83.185) (width 0.5) (layer "B.Cu") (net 3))
 (segment (start 160.015 90.17) (end 160.015 97.79) (width 0.5) (layer "B.Cu") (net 3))
 (segment (start 137.83 69.175) (end 137.83 72.14) (width 0.5) (layer "B.Cu") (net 3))
 (segment (start 139.06 102.87) (end 137.155 100.965) (width 0.5) (layer "B.Cu") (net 3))
 (segment (start 153.685 71.755) (end 149.855 71.755) (width 0.5) (layer "B.Cu") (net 3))
 (segment (start 152.4 83.185) (end 154.955 83.185) (width 0.5) (layer "B.Cu") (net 3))
 (segment (start 142.235 90.17) (end 142.235 88.245) (width 0.5) (layer "B.Cu") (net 3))
 (segment (start 143.715 71.755) (end 143.33 72.14) (width 0.5) (layer "B.Cu") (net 3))
 (segment (start 134.595 78.105) (end 134.615 78.085) (width 0.5) (layer "B.Cu") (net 3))
 (segment (start 154.955 87.63) (end 154.955 90.15) (width 0.5) (layer "B.Cu") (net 3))
 (segment (start 136.52 73.45) (end 137.83 72.14) (width 0.5) (layer "B.Cu") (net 3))
 (segment (start 161.92 99.695) (end 160.015 97.79) (width 0.5) (layer "B.Cu") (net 3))
 (segment (start 161.92 104.14) (end 161.92 99.695) (width 0.5) (layer "B.Cu") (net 3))
 (segment (start 147.315 104.775) (end 152.395 104.775) (width 0.5) (layer "B.Cu") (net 3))
 (segment (start 142.24 102.87) (end 139.06 102.87) (width 0.5) (layer "B.Cu") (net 3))
 (segment (start 161.285 104.775) (end 161.92 104.14) (width 0.5) (layer "B.Cu") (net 3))
 (segment (start 149.855 67.31) (end 139.695 67.31) (width 0.5) (layer "B.Cu") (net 3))
 (segment (start 132.08 107.315) (end 144.775 107.315) (width 0.5) (layer "B.Cu") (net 3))
 (segment (start 154.955 73.025) (end 153.685 71.755) (width 0.5) (layer "B.Cu") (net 3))
 (segment (start 154.935 90.17) (end 152.395 90.17) (width 0.5) (layer "B.Cu") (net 3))
 (segment (start 134.615 83.185) (end 134.615 88.240113) (width 0.5) (layer "B.Cu") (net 3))
 (segment (start 152.395 87.63) (end 154.955 87.63) (width 0.5) (layer "B.Cu") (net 3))
 (segment (start 136.52 78.085) (end 136.52 73.45) (width 0.5) (layer "B.Cu") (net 3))
 (segment (start 139.7 92.705) (end 142.235 90.17) (width 0.5) (layer "B.Cu") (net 3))
 (segment (start 152.395 102.87) (end 152.395 104.775) (width 0.5) (layer "B.Cu") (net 3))
 (segment (start 134.615 88.240113) (end 134.590113 88.265) (width 0.5) (layer "B.Cu") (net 3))
 (segment (start 154.955 90.15) (end 154.935 90.17) (width 0.5) (layer "B.Cu") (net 3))
 (segment (start 137.155 92.71) (end 139.7 92.71) (width 0.5) (layer "B.Cu") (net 3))
 (segment (start 129.535 78.105) (end 134.595 78.105) (width 0.5) (layer "B.Cu") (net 3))
 (segment (start 134.590113 90.145113) (end 137.155 92.71) (width 0.5) (layer "B.Cu") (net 3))
 (segment (start 149.855 71.755) (end 143.715 71.755) (width 0.5) (layer "B.Cu") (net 3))
 (segment (start 132.08 102.87) (end 132.08 107.315) (width 0.5) (layer "B.Cu") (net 3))
 (segment (start 134.615 78.085) (end 136.52 78.085) (width 0.5) (layer "B.Cu") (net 3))
 (segment (start 139.695 67.31) (end 137.83 69.175) (width 0.5) (layer "B.Cu") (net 3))
 (segment (start 134.615 95.245) (end 134.615 100.965) (width 0.5) (layer "B.Cu") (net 8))
 (segment (start 134.615 80.645) (end 132.075 83.185) (width 0.5) (layer "B.Cu") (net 8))
 (segment (start 160.02 73.03) (end 160.015 73.025) (width 0.5) (layer "B.Cu") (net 8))
 (segment (start 157.455 73.025) (end 160.015 73.025) (width 0.5) (layer "B.Cu") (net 8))
 (segment (start 161.285 107.315) (end 147.315 107.315) (width 0.5) (layer "B.Cu") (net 8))
 (segment (start 161.92 73.025) (end 160.025 73.025) (width 0.5) (layer "B.Cu") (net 8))
 (segment (start 149.86 95.25) (end 144.775 95.25) (width 0.5) (layer "B.Cu") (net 8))
 (segment (start 129.855 90.485) (end 126.995 87.625) (width 0.5) (layer "B.Cu") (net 8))
 (segment (start 160.02 75.565) (end 160.02 73.03) (width 0.5) (layer "B.Cu") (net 8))
 (segment (start 129.535 75.565) (end 134.595 75.565) (width 0.5) (layer "B.Cu") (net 8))
 (segment (start 126.995 78.105) (end 129.535 75.565) (width 0.5) (layer "B.Cu") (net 8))
 (segment (start 132.075 83.185) (end 132.075 88.265) (width 0.5) (layer "B.Cu") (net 8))
 (segment (start 163.825 104.775) (end 161.285 107.315) (width 0.5) (layer "B.Cu") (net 8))
 (segment (start 160.015 87.63) (end 162.555 90.17) (width 0.5) (layer "B.Cu") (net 8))
 (segment (start 163.825 91.44) (end 163.825 104.775) (width 0.5) (layer "B.Cu") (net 8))
 (segment (start 147.315 107.315) (end 144.775 104.775) (width 0.5) (layer "B.Cu") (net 8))
 (segment (start 166.365 74.295) (end 163.19 74.295) (width 0.5) (layer "B.Cu") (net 8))
 (segment (start 134.595 75.565) (end 134.615 75.585) (width 0.5) (layer "B.Cu") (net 8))
 (segment (start 126.995 87.625) (end 126.995 78.105) (width 0.5) (layer "B.Cu") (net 8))
 (segment (start 163.19 74.295) (end 161.92 73.025) (width 0.5) (layer "B.Cu") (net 8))
 (segment (start 162.555 90.17) (end 167.635 85.09) (width 0.5) (layer "B.Cu") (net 8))
 (segment (start 132.075 88.265) (end 129.855 90.485) (width 0.5) (layer "B.Cu") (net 8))
 (segment (start 132.08 92.71) (end 134.615 95.245) (width 0.5) (layer "B.Cu") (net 8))
 (segment (start 167.635 75.565) (end 166.365 74.295) (width 0.5) (layer "B.Cu") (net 8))
 (segment (start 144.775 104.775) (end 144.775 95.25) (width 0.5) (layer "B.Cu") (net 8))
 (segment (start 144.775 95.25) (end 142.24 95.25) (width 0.5) (layer "B.Cu") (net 8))
 (segment (start 132.08 92.71) (end 129.855 90.485) (width 0.5) (layer "B.Cu") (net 8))
 (segment (start 160.025 73.025) (end 160.02 73.03) (width 0.5) (layer "B.Cu") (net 8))
 (segment (start 162.555 90.17) (end 163.825 91.44) (width 0.5) (layer "B.Cu") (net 8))
 (segment (start 167.635 85.09) (end 167.635 75.565) (width 0.5) (layer "B.Cu") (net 8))
 (segment (start 138.425 104.775) (end 144.775 104.775) (width 0.5) (layer "B.Cu") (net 8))
 (segment (start 134.615 100.965) (end 138.425 104.775) (width 0.5) (layer "B.Cu") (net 8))
 (segment (start 160.015 85.725) (end 152.395 85.725) (width 0.5) (layer "F.Cu") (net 9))
 (via (at 152.395 85.725) (size 0.6) (drill 0.3) (layers "F.Cu" "B.Cu") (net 9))
 (via (at 160.015 85.725) (size 0.6) (drill 0.3) (layers "F.Cu" "B.Cu") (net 9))
 (segment (start 142.235 80.645) (end 142.235 85.745) (width 0.5) (layer "B.Cu") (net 9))
 (segment (start 149.855 82.55) (end 149.855 80.645) (width 0.5) (layer "B.Cu") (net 9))
 (segment (start 142.235 85.745) (end 139.610113 85.745) (width 0.5) (layer "B.Cu") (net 9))
 (segment (start 152.395 85.725) (end 152.375 85.745) (width 0.5) (layer "B.Cu") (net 9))
 (segment (start 160.02 83.185) (end 160.02 85.72) (width 0.5) (layer "B.Cu") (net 9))
 (segment (start 149.855 80.645) (end 152.4 80.645) (width 0.5) (layer "B.Cu") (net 9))
 (segment (start 149.855 82.55) (end 142.87 82.55) (width 0.5) (layer "B.Cu") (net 9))
 (segment (start 142.87 82.55) (end 142.235 83.185) (width 0.5) (layer "B.Cu") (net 9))
 (segment (start 152.375 85.745) (end 142.235 85.745) (width 0.5) (layer "B.Cu") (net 9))
 (segment (start 139.610113 85.745) (end 137.090113 88.265) (width 0.5) (layer "B.Cu") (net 9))
 (segment (start 160.02 85.72) (end 160.015 85.725) (width 0.5) (layer "B.Cu") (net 9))
 (segment (start 129.535 92.71) (end 129.535 97.785) (width 0.5) (layer "B.Cu") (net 12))
 (segment (start 129.535 97.785) (end 129.54 97.79) (width 0.5) (layer "B.Cu") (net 12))
 (segment (start 139.7 100.33) (end 142.24 100.33) (width 0.5) (layer "B.Cu") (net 19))
 (segment (start 139.7 97.79) (end 142.24 97.79) (width 0.5) (layer "B.Cu") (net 18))
 (segment (start 149.86 97.79) (end 152.395 97.79) (width 0.5) (layer "B.Cu") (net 5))
 (segment (start 149.86 100.33) (end 152.395 100.33) (width 0.5) (layer "B.Cu") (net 6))
 (via (at 129.535 102.87) (size 0.6) (drill 0.3) (layers "F.Cu" "B.Cu") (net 17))
 (segment (start 129.54 100.33) (end 126.365 103.505) (width 0.5) (layer "B.Cu") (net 16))
 (segment (start 126.365 103.505) (end 126.365 109.855) (width 0.5) (layer "B.Cu") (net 16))
 (segment (start 154.935 109.9485) (end 155.829 110.8425) (width 0.5) (layer "F.Cu") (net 15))
 (segment (start 154.935 102.89) (end 154.935 109.9485) (width 0.5) (layer "F.Cu") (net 15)))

